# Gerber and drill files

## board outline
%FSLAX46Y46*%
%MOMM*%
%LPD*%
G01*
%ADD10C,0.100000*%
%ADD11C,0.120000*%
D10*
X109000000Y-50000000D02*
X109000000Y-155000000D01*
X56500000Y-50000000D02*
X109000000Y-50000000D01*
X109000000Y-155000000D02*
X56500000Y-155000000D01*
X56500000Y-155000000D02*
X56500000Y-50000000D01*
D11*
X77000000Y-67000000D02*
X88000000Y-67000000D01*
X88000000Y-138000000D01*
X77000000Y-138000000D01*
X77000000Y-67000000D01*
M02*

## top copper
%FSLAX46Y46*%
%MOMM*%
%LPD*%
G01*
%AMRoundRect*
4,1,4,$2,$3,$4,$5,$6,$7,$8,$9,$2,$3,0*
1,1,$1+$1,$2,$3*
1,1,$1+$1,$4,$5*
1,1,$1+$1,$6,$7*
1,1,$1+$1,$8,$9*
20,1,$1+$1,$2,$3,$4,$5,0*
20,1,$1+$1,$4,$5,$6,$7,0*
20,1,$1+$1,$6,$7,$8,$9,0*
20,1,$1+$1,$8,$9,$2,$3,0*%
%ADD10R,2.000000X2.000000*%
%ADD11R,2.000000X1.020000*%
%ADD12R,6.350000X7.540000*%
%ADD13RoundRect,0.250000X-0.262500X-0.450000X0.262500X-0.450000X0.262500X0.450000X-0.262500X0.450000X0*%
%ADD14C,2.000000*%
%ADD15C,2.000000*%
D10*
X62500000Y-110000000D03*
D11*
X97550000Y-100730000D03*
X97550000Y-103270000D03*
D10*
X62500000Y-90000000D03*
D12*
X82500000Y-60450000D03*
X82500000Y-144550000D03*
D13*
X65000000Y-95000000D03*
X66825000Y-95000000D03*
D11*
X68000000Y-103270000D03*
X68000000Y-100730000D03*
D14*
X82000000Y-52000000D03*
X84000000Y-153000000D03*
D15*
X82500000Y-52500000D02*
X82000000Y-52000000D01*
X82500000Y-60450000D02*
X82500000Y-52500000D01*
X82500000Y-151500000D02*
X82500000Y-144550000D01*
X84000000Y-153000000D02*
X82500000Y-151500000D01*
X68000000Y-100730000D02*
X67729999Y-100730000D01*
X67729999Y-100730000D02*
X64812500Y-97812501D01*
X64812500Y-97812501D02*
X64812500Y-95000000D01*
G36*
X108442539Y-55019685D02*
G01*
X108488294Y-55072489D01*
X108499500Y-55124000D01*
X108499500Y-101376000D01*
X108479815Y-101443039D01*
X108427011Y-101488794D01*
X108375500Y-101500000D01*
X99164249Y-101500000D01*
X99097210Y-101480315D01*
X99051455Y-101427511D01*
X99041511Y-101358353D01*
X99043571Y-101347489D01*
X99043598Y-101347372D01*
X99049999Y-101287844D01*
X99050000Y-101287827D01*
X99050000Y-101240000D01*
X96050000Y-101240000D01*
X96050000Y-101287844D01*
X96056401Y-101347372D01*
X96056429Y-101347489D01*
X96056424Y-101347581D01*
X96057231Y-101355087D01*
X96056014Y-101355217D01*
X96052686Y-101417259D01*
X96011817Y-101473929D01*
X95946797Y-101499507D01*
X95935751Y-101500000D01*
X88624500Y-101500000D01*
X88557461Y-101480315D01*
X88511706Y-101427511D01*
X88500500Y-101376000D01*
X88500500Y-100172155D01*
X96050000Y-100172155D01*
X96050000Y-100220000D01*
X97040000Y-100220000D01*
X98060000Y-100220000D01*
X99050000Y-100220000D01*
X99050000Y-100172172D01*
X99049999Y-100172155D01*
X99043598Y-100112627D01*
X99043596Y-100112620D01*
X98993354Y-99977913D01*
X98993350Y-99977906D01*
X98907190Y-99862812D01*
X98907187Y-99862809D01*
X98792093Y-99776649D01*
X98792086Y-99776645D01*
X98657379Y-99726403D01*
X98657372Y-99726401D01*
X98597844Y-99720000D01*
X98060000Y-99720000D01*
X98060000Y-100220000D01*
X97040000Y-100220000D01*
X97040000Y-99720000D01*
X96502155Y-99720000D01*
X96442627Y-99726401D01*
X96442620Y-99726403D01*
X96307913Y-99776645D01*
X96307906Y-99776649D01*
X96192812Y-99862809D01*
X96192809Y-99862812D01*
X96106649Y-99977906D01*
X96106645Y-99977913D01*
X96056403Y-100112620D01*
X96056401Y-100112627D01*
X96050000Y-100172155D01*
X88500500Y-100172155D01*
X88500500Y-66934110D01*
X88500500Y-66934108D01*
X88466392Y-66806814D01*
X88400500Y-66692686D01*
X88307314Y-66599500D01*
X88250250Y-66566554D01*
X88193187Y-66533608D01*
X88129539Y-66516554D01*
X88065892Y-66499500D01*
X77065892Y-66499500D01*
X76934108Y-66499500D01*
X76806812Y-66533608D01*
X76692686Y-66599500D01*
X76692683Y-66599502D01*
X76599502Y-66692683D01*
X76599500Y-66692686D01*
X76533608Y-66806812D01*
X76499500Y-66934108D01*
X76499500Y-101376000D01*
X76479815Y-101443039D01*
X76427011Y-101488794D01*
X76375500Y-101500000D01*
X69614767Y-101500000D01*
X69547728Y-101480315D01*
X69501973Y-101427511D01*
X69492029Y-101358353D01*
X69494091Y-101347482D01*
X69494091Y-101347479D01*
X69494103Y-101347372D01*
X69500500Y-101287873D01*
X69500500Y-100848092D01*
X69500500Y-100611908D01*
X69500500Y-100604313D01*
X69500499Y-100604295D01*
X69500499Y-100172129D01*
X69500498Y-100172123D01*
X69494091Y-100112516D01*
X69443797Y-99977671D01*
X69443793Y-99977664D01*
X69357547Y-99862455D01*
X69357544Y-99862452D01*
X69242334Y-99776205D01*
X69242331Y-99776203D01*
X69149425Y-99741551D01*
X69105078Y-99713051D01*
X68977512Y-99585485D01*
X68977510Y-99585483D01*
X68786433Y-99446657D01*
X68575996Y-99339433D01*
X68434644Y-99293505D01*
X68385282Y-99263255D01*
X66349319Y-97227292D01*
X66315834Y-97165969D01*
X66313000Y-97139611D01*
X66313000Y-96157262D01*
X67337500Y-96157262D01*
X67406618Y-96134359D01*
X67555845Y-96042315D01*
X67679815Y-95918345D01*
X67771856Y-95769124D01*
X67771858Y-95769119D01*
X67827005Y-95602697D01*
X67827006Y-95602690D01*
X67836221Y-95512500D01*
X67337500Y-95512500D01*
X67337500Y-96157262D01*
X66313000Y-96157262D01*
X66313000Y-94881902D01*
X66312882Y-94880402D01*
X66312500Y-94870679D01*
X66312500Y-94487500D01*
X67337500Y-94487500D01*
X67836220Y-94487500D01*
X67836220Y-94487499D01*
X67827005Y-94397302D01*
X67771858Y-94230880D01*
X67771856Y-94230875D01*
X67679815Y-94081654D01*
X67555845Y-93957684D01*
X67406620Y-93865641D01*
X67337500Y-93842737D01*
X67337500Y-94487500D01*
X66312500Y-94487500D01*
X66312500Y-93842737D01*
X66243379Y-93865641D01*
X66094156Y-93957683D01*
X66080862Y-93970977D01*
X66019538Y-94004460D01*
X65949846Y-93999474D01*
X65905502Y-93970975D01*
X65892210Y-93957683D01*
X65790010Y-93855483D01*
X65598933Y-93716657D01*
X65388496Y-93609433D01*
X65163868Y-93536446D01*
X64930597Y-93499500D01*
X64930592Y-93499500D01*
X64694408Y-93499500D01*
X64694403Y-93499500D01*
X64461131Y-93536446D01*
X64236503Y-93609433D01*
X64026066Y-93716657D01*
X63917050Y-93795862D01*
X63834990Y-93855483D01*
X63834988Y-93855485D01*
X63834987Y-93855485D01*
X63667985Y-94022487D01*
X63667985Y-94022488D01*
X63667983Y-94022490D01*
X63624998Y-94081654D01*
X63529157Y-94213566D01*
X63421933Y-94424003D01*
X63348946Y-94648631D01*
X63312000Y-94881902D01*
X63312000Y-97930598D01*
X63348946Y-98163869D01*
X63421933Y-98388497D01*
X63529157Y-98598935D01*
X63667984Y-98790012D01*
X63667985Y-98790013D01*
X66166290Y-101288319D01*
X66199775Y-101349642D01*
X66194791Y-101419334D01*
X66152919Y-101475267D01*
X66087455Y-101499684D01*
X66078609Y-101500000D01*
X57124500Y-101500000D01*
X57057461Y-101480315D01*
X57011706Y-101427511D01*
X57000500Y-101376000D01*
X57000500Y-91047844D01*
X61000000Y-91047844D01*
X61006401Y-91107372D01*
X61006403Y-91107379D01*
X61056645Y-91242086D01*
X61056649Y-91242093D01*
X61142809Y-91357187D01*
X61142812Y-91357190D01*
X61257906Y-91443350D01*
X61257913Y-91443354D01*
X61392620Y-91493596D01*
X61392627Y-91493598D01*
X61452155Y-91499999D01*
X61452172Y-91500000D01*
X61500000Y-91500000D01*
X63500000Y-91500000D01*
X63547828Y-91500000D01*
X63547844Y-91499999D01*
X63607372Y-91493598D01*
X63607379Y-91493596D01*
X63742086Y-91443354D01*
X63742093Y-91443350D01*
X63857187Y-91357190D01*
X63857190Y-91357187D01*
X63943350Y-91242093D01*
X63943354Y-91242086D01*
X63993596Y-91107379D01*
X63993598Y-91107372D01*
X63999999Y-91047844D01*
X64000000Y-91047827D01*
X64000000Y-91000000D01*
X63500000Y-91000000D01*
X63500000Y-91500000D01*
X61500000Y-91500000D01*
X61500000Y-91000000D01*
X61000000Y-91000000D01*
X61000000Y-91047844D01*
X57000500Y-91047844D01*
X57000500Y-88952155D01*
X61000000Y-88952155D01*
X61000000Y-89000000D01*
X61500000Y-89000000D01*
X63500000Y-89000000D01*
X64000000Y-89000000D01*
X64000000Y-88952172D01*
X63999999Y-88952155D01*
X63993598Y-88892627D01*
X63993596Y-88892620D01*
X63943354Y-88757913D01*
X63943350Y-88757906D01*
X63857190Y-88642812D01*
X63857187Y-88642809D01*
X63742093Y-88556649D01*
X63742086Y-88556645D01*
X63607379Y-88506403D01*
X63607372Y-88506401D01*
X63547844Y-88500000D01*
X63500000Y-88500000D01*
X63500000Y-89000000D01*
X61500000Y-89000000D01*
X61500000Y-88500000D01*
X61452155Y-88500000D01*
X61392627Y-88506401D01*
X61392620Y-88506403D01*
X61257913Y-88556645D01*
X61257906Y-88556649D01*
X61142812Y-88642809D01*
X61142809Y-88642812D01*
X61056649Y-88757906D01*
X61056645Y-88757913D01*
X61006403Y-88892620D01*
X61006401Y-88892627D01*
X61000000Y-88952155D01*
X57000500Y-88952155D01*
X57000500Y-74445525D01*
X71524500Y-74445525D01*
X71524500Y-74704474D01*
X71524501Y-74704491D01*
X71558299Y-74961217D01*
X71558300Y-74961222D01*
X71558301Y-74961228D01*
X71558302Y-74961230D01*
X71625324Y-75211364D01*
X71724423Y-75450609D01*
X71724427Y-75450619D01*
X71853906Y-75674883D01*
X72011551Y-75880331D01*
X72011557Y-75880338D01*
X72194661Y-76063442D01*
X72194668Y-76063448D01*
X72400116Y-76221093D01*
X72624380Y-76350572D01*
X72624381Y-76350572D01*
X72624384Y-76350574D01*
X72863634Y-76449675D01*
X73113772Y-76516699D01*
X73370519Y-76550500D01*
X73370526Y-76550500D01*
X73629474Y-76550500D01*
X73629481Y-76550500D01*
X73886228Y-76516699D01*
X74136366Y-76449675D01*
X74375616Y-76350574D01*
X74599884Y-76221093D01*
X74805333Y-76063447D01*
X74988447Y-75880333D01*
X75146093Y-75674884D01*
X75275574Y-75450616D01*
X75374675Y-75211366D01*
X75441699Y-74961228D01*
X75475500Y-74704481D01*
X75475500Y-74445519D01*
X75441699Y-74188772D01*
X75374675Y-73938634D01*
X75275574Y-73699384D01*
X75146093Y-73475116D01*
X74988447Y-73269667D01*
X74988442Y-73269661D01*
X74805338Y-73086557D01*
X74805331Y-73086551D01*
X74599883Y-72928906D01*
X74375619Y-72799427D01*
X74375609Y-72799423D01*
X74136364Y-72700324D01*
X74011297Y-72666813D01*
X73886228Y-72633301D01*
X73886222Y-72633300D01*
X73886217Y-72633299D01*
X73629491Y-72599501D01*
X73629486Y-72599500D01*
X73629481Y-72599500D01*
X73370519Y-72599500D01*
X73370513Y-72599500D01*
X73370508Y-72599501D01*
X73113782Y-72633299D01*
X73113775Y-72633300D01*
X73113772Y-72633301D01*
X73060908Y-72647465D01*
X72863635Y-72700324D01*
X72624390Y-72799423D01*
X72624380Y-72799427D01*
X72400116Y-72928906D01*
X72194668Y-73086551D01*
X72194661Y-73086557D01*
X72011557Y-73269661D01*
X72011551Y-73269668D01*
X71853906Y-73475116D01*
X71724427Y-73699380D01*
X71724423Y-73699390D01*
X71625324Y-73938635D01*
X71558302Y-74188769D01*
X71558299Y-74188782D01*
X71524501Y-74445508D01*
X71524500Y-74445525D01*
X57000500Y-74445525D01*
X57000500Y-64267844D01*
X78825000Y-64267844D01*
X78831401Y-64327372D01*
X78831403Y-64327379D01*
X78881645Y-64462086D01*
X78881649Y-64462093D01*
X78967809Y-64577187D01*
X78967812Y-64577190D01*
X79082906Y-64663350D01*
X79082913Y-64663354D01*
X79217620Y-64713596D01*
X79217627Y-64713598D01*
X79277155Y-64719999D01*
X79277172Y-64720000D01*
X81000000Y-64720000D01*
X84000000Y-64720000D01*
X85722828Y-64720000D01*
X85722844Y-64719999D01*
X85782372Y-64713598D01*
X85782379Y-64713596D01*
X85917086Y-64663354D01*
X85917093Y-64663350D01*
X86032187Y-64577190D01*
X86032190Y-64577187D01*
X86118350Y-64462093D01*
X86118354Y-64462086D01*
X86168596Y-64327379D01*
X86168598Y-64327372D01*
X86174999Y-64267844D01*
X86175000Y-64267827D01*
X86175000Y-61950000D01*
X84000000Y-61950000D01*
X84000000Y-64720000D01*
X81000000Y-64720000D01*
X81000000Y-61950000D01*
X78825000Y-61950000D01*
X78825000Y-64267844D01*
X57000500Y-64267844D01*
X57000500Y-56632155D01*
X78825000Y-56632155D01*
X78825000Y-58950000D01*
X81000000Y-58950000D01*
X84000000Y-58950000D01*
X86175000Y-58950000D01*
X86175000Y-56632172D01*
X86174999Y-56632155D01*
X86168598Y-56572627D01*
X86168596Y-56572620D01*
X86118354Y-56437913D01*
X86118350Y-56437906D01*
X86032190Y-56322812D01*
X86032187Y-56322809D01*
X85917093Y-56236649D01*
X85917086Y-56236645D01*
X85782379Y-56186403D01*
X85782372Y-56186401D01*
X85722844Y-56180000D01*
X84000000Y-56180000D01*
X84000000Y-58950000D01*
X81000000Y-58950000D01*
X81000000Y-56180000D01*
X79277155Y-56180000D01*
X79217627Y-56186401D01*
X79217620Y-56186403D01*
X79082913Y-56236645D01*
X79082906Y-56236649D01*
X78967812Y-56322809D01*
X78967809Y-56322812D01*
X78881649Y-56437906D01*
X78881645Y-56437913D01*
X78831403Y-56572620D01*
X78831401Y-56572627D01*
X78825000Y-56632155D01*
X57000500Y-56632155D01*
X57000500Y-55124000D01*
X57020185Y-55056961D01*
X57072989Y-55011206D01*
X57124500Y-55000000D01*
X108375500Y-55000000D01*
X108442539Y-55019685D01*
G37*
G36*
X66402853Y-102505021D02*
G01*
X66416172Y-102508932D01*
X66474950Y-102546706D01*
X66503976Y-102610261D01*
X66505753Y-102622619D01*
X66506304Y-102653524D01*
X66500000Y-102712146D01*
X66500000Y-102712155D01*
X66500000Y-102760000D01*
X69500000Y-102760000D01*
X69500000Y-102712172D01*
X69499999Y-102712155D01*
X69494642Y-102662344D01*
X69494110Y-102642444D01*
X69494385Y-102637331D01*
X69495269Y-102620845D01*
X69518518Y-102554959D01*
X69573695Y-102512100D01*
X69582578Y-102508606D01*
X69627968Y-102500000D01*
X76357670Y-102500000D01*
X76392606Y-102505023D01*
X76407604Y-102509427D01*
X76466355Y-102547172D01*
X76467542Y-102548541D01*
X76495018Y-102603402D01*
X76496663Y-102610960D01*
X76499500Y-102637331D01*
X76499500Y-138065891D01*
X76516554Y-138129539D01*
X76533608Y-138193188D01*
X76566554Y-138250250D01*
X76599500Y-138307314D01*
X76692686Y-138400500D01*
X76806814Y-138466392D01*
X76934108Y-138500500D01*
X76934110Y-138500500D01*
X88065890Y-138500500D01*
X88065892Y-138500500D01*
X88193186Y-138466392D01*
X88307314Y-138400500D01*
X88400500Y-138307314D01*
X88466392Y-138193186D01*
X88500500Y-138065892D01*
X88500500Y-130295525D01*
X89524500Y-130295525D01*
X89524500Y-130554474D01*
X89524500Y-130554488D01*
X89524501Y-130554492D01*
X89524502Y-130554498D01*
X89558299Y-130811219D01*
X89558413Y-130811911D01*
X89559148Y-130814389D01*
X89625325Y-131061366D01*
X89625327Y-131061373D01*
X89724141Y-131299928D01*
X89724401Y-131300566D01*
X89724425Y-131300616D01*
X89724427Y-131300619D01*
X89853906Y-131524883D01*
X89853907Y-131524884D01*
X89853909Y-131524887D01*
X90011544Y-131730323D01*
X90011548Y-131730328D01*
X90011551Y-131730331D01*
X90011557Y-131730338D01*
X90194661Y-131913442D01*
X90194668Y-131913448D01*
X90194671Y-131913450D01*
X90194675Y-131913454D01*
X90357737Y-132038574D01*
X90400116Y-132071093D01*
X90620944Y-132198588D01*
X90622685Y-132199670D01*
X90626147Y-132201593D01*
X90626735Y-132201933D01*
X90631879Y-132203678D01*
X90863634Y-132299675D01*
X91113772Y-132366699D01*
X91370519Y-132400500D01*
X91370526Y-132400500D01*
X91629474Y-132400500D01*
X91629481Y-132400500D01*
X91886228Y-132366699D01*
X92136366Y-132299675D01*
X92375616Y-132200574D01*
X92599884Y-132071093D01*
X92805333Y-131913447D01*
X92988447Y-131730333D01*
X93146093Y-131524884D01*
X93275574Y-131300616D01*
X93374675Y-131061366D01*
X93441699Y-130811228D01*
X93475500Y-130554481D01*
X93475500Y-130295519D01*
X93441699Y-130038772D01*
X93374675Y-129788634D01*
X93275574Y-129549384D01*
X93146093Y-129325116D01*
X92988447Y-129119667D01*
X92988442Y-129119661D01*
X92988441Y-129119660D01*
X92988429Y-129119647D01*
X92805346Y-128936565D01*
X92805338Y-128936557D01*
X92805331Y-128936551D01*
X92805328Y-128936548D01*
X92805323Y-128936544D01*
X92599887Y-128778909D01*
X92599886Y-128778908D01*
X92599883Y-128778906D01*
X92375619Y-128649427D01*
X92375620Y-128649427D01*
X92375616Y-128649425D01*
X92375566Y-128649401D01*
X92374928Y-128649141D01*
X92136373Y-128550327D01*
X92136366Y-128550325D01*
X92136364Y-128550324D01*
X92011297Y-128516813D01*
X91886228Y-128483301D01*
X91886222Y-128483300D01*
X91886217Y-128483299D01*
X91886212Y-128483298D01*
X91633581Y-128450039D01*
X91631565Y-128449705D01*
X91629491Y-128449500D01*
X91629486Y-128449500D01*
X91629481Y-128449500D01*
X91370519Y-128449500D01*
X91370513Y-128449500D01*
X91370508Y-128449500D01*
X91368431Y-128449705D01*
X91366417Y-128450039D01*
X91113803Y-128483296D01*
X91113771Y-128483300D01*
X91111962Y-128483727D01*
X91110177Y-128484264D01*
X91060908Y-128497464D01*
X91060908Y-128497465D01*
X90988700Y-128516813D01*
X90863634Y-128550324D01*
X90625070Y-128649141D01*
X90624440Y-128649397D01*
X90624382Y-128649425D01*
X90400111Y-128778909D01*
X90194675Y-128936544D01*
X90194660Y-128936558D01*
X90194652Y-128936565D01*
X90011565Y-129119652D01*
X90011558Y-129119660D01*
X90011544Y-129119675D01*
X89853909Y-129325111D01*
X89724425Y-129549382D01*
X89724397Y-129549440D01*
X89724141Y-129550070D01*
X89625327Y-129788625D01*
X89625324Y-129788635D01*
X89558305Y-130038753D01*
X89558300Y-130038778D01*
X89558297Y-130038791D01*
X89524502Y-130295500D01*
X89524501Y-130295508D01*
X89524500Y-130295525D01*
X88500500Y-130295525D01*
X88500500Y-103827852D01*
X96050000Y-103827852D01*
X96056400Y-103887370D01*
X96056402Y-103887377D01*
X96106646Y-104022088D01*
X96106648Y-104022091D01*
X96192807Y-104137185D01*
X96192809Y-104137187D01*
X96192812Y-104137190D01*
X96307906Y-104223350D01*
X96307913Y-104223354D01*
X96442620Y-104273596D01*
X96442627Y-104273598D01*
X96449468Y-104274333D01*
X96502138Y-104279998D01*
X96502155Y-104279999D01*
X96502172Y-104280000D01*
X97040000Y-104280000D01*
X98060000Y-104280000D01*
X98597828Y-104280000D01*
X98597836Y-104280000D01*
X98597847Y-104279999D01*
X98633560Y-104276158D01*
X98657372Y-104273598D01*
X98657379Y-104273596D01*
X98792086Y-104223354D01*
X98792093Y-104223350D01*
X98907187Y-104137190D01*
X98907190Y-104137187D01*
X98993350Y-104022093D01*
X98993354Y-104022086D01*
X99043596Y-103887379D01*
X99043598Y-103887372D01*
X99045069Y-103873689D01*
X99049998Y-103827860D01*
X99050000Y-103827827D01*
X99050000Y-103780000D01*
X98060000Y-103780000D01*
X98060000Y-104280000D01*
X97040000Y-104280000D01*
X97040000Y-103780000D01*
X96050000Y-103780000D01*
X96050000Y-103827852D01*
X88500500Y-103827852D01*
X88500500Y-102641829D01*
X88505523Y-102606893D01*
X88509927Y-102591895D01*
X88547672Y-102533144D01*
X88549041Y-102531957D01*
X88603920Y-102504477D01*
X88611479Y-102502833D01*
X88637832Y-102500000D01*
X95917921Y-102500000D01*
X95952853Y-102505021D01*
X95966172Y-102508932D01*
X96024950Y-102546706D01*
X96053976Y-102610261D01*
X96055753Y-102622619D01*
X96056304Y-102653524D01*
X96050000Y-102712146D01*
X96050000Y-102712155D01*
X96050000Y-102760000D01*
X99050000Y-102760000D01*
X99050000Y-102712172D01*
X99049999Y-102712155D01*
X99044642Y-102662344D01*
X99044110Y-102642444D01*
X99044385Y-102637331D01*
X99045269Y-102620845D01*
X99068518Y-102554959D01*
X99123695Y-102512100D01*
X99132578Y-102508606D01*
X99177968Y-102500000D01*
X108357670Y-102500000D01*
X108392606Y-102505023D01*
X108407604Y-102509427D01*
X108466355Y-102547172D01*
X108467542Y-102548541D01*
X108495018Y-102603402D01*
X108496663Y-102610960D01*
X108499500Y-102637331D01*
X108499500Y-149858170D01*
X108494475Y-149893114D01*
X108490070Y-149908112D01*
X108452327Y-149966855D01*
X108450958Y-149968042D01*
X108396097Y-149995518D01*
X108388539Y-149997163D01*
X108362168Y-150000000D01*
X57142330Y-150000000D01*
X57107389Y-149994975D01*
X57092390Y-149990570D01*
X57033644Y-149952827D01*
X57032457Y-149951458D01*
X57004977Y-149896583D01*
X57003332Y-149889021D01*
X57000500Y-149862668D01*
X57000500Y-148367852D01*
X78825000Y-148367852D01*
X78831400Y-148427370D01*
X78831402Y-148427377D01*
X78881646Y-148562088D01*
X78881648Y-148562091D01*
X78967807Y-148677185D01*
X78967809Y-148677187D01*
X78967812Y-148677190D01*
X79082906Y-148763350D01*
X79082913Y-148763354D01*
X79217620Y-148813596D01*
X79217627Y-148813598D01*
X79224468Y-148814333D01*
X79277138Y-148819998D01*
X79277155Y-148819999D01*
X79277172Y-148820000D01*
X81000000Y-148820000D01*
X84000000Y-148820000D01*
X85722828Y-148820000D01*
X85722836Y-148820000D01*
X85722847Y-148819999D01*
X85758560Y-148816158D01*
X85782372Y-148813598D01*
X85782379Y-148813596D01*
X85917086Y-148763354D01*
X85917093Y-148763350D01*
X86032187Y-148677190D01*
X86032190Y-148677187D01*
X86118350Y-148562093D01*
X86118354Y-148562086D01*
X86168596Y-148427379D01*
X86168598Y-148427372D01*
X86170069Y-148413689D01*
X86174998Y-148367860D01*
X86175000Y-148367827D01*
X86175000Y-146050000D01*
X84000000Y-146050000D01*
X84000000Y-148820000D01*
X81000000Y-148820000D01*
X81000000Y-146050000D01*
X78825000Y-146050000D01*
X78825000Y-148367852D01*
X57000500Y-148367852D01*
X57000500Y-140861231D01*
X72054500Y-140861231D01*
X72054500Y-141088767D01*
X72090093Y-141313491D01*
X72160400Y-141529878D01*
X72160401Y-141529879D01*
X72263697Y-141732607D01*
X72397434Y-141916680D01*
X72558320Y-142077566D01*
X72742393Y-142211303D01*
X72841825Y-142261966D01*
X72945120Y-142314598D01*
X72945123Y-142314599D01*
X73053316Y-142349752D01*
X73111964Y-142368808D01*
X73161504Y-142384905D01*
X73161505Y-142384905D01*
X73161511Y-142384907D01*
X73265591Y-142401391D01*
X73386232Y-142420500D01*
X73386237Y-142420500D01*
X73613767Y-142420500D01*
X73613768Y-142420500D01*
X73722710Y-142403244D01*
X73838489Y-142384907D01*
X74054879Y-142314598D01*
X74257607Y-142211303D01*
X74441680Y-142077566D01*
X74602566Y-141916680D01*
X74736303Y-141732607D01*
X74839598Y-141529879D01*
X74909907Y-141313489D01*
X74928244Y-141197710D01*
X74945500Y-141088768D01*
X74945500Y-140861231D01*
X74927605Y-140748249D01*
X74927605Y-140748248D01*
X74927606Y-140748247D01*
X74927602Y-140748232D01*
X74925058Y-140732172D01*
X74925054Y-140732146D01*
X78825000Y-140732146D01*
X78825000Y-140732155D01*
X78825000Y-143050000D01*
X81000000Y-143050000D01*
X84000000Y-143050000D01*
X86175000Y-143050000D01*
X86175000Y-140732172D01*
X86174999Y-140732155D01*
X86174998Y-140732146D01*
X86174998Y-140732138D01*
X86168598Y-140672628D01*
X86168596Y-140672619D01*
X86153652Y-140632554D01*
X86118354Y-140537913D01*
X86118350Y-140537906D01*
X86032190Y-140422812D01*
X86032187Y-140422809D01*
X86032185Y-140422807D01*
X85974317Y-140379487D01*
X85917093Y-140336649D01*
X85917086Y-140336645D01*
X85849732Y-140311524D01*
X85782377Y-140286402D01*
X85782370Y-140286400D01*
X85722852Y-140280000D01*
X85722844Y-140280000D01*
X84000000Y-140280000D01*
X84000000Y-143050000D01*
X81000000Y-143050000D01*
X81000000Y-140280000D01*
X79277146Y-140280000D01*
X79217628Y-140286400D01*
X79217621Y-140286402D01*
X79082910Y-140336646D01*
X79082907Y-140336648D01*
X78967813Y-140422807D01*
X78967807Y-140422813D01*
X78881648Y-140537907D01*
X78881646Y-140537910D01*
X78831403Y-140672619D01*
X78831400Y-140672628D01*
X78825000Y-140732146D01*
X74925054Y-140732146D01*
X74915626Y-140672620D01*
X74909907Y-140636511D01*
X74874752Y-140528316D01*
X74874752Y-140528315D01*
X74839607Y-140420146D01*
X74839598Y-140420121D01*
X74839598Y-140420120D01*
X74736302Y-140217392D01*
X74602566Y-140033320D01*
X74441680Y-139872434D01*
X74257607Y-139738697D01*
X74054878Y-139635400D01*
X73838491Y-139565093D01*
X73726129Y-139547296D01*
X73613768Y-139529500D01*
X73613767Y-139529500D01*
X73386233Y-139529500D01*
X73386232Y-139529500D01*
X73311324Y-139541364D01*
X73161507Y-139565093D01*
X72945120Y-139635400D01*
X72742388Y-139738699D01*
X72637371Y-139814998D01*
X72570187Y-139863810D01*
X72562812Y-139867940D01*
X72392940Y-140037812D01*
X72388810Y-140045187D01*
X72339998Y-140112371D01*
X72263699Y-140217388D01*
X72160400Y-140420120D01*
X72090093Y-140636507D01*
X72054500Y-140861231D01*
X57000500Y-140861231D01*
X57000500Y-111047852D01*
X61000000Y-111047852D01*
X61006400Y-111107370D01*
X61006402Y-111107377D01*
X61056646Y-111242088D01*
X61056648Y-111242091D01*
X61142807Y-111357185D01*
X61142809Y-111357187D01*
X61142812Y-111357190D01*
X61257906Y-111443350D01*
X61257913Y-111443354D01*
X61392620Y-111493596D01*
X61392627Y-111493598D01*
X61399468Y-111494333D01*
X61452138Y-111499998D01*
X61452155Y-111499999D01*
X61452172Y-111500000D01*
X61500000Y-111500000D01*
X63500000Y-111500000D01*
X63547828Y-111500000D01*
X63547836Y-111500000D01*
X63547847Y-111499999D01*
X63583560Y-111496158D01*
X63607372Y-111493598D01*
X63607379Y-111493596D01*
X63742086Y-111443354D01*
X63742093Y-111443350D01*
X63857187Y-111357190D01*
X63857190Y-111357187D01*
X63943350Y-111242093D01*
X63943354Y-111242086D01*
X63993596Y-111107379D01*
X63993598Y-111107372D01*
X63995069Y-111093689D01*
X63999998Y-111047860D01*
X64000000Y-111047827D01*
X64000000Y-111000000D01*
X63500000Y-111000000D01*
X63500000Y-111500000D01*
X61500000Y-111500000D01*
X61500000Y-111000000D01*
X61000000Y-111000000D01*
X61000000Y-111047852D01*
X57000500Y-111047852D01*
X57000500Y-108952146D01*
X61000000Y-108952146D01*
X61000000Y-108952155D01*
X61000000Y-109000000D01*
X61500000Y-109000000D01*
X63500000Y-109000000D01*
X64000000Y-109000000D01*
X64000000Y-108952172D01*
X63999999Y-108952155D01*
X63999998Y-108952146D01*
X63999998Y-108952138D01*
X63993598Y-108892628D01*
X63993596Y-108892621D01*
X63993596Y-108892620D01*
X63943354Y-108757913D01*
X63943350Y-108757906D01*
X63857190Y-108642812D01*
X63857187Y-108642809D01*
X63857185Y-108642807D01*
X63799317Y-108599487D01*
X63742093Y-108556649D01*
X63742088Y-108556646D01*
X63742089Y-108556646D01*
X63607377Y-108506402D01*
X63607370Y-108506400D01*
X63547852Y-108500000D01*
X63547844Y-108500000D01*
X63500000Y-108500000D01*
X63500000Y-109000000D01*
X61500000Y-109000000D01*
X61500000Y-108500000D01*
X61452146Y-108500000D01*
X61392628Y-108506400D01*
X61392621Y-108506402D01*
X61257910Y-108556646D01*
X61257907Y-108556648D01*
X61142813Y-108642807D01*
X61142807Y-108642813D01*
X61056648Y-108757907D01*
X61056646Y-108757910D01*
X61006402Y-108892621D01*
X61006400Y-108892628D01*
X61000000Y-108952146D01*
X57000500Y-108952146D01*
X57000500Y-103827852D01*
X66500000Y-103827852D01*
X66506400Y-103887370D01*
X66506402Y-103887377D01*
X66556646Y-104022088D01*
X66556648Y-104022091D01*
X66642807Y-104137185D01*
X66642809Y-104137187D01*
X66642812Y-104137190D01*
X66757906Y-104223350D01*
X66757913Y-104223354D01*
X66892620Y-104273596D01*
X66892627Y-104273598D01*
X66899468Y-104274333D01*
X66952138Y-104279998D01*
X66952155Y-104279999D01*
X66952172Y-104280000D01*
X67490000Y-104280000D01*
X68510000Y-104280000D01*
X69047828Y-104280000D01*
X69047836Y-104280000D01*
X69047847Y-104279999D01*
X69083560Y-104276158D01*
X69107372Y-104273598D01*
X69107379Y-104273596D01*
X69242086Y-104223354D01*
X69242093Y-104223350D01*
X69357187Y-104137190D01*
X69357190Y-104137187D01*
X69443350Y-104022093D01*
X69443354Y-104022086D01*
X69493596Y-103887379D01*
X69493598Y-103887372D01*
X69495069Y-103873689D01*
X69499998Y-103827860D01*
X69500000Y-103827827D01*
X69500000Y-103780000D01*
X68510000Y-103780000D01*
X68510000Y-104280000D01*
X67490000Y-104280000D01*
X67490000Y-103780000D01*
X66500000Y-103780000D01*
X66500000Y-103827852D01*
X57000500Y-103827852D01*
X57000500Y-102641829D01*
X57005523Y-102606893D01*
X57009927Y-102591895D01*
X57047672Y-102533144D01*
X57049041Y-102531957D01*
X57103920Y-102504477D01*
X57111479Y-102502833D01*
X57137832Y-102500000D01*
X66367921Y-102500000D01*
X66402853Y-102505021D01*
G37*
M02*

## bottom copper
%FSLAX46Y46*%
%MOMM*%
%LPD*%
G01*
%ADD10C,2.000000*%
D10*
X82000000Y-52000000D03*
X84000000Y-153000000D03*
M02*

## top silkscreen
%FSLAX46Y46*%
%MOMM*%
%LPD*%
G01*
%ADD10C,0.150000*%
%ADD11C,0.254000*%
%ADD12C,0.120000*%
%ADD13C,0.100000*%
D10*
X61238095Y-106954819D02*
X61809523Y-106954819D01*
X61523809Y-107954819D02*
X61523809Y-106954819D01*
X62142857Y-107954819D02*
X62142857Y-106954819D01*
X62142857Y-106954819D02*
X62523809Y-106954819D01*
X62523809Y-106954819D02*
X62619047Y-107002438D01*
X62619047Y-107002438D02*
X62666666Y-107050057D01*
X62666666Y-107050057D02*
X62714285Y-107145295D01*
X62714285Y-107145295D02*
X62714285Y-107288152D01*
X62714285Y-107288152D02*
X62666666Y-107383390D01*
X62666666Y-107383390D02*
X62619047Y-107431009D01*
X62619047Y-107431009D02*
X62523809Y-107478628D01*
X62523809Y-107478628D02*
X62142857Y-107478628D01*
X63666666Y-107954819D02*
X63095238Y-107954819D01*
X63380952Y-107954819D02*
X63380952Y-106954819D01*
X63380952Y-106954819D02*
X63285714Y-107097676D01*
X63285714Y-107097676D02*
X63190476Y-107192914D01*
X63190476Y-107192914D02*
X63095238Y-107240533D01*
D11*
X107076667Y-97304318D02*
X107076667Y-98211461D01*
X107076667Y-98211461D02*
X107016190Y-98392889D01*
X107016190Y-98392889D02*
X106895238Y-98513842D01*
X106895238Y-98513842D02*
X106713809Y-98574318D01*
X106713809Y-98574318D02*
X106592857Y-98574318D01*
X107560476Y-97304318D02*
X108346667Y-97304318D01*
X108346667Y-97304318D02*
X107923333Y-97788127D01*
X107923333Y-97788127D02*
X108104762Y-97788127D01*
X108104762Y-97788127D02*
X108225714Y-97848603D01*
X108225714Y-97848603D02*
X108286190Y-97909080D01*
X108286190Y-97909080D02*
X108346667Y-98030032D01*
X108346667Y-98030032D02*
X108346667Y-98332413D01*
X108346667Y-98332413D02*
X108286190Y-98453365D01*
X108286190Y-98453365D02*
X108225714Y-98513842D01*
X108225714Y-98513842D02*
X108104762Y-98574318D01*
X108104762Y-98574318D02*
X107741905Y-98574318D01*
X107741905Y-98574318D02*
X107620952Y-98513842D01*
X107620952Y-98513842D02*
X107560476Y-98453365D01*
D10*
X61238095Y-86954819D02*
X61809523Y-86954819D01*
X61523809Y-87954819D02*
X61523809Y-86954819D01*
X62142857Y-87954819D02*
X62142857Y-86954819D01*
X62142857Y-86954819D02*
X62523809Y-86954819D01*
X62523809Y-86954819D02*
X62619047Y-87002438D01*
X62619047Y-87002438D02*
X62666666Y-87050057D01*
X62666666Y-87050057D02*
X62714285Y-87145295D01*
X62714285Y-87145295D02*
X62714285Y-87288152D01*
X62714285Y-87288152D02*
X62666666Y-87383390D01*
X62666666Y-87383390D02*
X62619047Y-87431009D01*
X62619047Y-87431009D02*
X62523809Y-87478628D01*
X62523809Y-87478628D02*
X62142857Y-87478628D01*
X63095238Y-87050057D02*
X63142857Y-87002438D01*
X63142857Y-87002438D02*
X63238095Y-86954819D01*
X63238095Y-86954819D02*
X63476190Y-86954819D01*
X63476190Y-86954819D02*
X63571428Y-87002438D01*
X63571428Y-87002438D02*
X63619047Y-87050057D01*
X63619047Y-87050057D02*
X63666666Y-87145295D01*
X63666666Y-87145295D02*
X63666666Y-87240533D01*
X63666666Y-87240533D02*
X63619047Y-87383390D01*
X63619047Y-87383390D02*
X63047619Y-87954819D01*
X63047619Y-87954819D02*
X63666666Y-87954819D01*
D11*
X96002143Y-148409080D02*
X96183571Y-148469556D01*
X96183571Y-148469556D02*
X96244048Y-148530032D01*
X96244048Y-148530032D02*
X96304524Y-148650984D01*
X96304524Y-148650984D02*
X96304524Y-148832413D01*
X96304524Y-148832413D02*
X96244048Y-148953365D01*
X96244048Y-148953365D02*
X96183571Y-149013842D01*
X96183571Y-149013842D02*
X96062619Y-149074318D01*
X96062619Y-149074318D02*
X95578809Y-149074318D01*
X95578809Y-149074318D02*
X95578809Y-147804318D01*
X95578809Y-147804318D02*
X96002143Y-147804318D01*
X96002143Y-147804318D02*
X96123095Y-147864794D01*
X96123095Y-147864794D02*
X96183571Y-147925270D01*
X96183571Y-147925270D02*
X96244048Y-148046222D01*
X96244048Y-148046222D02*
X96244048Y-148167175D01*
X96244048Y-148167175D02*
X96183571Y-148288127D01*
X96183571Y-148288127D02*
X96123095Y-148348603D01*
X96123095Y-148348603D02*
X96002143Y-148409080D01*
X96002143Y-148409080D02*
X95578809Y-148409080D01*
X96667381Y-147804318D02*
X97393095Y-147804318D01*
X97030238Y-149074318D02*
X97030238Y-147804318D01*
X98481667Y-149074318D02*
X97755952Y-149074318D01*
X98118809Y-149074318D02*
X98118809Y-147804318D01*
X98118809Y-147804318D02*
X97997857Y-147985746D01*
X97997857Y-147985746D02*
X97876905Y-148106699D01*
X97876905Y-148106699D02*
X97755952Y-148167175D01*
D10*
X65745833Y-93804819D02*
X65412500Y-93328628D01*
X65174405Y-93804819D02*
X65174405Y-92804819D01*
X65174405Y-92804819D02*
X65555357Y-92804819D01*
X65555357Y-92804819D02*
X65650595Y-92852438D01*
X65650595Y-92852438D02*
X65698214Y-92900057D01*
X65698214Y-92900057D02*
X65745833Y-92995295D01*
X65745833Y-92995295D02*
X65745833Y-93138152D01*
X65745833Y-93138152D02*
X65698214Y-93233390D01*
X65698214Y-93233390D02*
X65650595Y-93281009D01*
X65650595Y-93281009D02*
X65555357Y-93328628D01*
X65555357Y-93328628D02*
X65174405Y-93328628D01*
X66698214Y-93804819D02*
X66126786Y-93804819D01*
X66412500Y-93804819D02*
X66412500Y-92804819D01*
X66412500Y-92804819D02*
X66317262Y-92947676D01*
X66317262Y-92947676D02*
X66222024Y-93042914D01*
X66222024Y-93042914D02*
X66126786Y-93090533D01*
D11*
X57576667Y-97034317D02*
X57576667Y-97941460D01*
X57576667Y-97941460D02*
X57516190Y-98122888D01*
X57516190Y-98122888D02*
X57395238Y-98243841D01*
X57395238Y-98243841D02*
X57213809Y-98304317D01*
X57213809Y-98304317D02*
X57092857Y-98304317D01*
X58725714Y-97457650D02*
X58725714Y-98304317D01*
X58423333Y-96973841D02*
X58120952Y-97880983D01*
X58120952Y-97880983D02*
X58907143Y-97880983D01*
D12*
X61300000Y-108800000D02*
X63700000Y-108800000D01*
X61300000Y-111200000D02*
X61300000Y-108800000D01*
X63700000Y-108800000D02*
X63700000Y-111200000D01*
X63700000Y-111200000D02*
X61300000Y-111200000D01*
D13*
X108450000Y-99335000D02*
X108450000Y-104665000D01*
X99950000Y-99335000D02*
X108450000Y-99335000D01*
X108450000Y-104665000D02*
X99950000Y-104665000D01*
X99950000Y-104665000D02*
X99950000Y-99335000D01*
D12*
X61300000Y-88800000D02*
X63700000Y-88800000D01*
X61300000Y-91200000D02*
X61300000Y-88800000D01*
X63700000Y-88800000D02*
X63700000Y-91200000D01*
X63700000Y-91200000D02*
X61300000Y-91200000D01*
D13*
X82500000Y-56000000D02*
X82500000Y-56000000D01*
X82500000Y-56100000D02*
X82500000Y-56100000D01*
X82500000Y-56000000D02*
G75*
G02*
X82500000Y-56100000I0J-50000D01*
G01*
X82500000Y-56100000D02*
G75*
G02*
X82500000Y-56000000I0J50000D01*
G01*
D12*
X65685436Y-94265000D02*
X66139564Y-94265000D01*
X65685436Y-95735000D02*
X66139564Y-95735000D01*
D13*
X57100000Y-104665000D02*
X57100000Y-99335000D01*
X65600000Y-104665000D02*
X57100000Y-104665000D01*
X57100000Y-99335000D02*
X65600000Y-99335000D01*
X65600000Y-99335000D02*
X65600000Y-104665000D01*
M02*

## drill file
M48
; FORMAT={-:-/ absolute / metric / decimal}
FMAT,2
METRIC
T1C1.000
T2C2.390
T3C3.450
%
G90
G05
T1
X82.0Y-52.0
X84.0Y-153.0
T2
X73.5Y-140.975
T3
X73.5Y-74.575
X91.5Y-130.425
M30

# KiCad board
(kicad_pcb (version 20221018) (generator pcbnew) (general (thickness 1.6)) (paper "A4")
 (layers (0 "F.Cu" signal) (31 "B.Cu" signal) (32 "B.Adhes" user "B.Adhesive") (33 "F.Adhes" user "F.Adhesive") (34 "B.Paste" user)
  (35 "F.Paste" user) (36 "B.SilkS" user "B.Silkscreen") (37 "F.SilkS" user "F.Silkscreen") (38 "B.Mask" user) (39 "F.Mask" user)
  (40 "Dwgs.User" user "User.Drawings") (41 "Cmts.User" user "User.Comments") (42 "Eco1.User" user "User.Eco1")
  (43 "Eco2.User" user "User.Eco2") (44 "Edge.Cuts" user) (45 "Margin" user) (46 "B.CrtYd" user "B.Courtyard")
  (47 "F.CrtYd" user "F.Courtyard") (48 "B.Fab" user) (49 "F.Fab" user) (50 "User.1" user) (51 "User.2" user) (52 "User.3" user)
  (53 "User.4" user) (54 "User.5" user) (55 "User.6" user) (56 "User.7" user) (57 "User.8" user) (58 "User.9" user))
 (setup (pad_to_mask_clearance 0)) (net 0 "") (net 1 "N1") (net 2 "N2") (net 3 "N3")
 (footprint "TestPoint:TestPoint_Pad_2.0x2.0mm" (layer "F.Cu") (at 62.5 110)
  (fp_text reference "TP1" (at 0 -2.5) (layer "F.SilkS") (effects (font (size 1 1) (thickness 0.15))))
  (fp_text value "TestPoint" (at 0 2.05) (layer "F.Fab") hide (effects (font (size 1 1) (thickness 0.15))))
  (fp_line (start -1.2 -1.2) (end 1.2 -1.2) (stroke (width 0.12) (type solid)) (layer "F.SilkS"))
  (fp_line (start -1.2 1.2) (end -1.2 -1.2) (stroke (width 0.12) (type solid)) (layer "F.SilkS"))
  (fp_line (start 1.2 -1.2) (end 1.2 1.2) (stroke (width 0.12) (type solid)) (layer "F.SilkS"))
  (fp_line (start 1.2 1.2) (end -1.2 1.2) (stroke (width 0.12) (type solid)) (layer "F.SilkS"))
  (pad "1" smd rect (at 0 0) (size 2 2) (layers "F.Cu" "F.Mask") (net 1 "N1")))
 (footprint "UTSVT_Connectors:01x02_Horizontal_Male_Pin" (layer "F.Cu") (at 103 102 -90)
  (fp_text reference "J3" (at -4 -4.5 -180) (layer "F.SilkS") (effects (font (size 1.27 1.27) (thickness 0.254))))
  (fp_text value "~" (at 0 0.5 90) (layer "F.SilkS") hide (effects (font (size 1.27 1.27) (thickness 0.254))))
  (fp_line (start -2.665 -5.45) (end 2.665 -5.45) (stroke (width 0.1) (type solid)) (layer "F.SilkS"))
  (fp_line (start -2.665 3.05) (end -2.665 -5.45) (stroke (width 0.1) (type solid)) (layer "F.SilkS"))
  (fp_line (start 2.665 -5.45) (end 2.665 3.05) (stroke (width 0.1) (type solid)) (layer "F.SilkS"))
  (fp_line (start 2.665 3.05) (end -2.665 3.05) (stroke (width 0.1) (type solid)) (layer "F.SilkS"))
  (pad "1" smd rect (at -1.27 5.45 270) (size 1.02 2) (layers "F.Cu" "F.Paste" "F.Mask") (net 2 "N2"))
  (pad "2" smd rect (at 1.27 5.45 270) (size 1.02 2) (layers "F.Cu" "F.Paste" "F.Mask") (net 1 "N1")))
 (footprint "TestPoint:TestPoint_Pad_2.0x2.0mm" (layer "F.Cu") (at 62.5 90)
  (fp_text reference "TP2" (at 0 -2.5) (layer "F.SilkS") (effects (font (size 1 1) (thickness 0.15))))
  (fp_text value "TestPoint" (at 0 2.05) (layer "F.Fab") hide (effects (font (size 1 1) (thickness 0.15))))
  (fp_line (start -1.2 -1.2) (end 1.2 -1.2) (stroke (width 0.12) (type solid)) (layer "F.SilkS"))
  (fp_line (start -1.2 1.2) (end -1.2 -1.2) (stroke (width 0.12) (type solid)) (layer "F.SilkS"))
  (fp_line (start 1.2 -1.2) (end 1.2 1.2) (stroke (width 0.12) (type solid)) (layer "F.SilkS"))
  (fp_line (start 1.2 1.2) (end -1.2 1.2) (stroke (width 0.12) (type solid)) (layer "F.SilkS"))
  (pad "1" smd rect (at 0 0) (size 2 2) (layers "F.Cu" "F.Mask") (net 2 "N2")))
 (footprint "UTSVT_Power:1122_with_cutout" (layer "F.Cu") (at 82.5 102.5 -90)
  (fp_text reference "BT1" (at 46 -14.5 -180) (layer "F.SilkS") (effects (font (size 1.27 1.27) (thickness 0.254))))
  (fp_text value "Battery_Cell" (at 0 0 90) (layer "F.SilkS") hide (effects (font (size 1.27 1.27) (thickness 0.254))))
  (fp_line (start -46.5 0) (end -46.5 0) (stroke (width 0.1) (type solid)) (layer "F.SilkS"))
  (fp_line (start -46.4 0) (end -46.4 0) (stroke (width 0.1) (type solid)) (layer "F.SilkS"))
  (fp_arc (start -46.5 0) (mid -46.45 -0.05) (end -46.4 0) (stroke (width 0.1) (type solid)) (layer "F.SilkS"))
  (fp_arc (start -46.4 0) (mid -46.45 0.05) (end -46.5 0) (stroke (width 0.1) (type solid)) (layer "F.SilkS"))
  (fp_rect (start -35.5 -5.5) (end 35.5 5.5) (stroke (width 0.12) (type solid)) (fill none) (layer "Edge.Cuts"))
  (pad "" np_thru_hole circle (at -27.925 9 270) (size 3.45 3.45) (drill 3.45) (layers "*.Cu" "*.Mask"))
  (pad "" np_thru_hole circle (at 27.925 -9 270) (size 3.45 3.45) (drill 3.45) (layers "*.Cu" "*.Mask"))
  (pad "" np_thru_hole circle (at 38.475 9 270) (size 2.39 2.39) (drill 2.39) (layers "*.Cu" "*.Mask"))
  (pad "1" smd rect (at -42.05 0) (size 6.35 7.54) (layers "F.Cu" "F.Paste" "F.Mask") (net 2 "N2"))
  (pad "2" smd rect (at 42.05 0) (size 6.35 7.54) (layers "F.Cu" "F.Paste" "F.Mask") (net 1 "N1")))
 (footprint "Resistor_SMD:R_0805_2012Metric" (layer "F.Cu") (at 65.9125 95)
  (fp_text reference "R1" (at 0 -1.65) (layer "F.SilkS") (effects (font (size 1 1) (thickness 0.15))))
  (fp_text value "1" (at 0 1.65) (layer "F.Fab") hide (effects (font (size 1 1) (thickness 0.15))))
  (fp_line (start -0.227064 -0.735) (end 0.227064 -0.735) (stroke (width 0.12) (type solid)) (layer "F.SilkS"))
  (fp_line (start -0.227064 0.735) (end 0.227064 0.735) (stroke (width 0.12) (type solid)) (layer "F.SilkS"))
  (pad "1" smd roundrect (at -0.9125 0) (size 1.025 1.4) (layers "F.Cu" "F.Paste" "F.Mask") (roundrect_rratio 0.243902) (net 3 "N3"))
  (pad "2" smd roundrect (at 0.9125 0) (size 1.025 1.4) (layers "F.Cu" "F.Paste" "F.Mask") (roundrect_rratio 0.243902) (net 2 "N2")))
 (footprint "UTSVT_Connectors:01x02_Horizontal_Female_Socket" (layer "F.Cu") (at 62.55 102 90)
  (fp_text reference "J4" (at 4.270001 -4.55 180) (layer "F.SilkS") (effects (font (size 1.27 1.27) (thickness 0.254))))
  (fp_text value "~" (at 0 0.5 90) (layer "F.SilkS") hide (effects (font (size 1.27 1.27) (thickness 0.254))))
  (fp_line (start -2.665 -5.45) (end 2.665 -5.45) (stroke (width 0.1) (type solid)) (layer "F.SilkS"))
  (fp_line (start -2.665 3.05) (end -2.665 -5.45) (stroke (width 0.1) (type solid)) (layer "F.SilkS"))
  (fp_line (start 2.665 -5.45) (end 2.665 3.05) (stroke (width 0.1) (type solid)) (layer "F.SilkS"))
  (fp_line (start 2.665 3.05) (end -2.665 3.05) (stroke (width 0.1) (type solid)) (layer "F.SilkS"))
  (pad "1" smd rect (at -1.27 5.45 90) (size 1.02 2) (layers "F.Cu" "F.Paste" "F.Mask") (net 1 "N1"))
  (pad "2" smd rect (at 1.27 5.45 90) (size 1.02 2) (layers "F.Cu" "F.Paste" "F.Mask") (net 3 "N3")))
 (gr_line (start 109 50) (end 109 155) (stroke (width 0.1) (type default)) (layer "Edge.Cuts"))
 (gr_line (start 56.5 50) (end 109 50) (stroke (width 0.1) (type default)) (layer "Edge.Cuts"))
 (gr_line (start 109 155) (end 56.5 155) (stroke (width 0.1) (type default)) (layer "Edge.Cuts"))
 (gr_line (start 56.5 155) (end 56.5 50) (stroke (width 0.1) (type default)) (layer "Edge.Cuts"))
 (segment (start 82.5 52.5) (end 82 52) (width 2) (layer "F.Cu") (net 2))
 (segment (start 82.5 60.45) (end 82.5 52.5) (width 2) (layer "F.Cu") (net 2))
 (via (at 82 52) (size 2) (drill 1) (layers "F.Cu" "B.Cu") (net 2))
 (segment (start 82.5 151.5) (end 82.5 144.55) (width 2) (layer "F.Cu") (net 1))
 (segment (start 84 153) (end 82.5 151.5) (width 2) (layer "F.Cu") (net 1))
 (via (at 84 153) (size 2) (drill 1) (layers "F.Cu" "B.Cu") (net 1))
 (segment (start 68 100.73) (end 67.729999 100.73) (width 2) (layer "F.Cu") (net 3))
 (segment (start 67.729999 100.73) (end 64.8125 97.812501) (width 2) (layer "F.Cu") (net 3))
 (segment (start 64.8125 97.812501) (end 64.8125 95) (width 2) (layer "F.Cu") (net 3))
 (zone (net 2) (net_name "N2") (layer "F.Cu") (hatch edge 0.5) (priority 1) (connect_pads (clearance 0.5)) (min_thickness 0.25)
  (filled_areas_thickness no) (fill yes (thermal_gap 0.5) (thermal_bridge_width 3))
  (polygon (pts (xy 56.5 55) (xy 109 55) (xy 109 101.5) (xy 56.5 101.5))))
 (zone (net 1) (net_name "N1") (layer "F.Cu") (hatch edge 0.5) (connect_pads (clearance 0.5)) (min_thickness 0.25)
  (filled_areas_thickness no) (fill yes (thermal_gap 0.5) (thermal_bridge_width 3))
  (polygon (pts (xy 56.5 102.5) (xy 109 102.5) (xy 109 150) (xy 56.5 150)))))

